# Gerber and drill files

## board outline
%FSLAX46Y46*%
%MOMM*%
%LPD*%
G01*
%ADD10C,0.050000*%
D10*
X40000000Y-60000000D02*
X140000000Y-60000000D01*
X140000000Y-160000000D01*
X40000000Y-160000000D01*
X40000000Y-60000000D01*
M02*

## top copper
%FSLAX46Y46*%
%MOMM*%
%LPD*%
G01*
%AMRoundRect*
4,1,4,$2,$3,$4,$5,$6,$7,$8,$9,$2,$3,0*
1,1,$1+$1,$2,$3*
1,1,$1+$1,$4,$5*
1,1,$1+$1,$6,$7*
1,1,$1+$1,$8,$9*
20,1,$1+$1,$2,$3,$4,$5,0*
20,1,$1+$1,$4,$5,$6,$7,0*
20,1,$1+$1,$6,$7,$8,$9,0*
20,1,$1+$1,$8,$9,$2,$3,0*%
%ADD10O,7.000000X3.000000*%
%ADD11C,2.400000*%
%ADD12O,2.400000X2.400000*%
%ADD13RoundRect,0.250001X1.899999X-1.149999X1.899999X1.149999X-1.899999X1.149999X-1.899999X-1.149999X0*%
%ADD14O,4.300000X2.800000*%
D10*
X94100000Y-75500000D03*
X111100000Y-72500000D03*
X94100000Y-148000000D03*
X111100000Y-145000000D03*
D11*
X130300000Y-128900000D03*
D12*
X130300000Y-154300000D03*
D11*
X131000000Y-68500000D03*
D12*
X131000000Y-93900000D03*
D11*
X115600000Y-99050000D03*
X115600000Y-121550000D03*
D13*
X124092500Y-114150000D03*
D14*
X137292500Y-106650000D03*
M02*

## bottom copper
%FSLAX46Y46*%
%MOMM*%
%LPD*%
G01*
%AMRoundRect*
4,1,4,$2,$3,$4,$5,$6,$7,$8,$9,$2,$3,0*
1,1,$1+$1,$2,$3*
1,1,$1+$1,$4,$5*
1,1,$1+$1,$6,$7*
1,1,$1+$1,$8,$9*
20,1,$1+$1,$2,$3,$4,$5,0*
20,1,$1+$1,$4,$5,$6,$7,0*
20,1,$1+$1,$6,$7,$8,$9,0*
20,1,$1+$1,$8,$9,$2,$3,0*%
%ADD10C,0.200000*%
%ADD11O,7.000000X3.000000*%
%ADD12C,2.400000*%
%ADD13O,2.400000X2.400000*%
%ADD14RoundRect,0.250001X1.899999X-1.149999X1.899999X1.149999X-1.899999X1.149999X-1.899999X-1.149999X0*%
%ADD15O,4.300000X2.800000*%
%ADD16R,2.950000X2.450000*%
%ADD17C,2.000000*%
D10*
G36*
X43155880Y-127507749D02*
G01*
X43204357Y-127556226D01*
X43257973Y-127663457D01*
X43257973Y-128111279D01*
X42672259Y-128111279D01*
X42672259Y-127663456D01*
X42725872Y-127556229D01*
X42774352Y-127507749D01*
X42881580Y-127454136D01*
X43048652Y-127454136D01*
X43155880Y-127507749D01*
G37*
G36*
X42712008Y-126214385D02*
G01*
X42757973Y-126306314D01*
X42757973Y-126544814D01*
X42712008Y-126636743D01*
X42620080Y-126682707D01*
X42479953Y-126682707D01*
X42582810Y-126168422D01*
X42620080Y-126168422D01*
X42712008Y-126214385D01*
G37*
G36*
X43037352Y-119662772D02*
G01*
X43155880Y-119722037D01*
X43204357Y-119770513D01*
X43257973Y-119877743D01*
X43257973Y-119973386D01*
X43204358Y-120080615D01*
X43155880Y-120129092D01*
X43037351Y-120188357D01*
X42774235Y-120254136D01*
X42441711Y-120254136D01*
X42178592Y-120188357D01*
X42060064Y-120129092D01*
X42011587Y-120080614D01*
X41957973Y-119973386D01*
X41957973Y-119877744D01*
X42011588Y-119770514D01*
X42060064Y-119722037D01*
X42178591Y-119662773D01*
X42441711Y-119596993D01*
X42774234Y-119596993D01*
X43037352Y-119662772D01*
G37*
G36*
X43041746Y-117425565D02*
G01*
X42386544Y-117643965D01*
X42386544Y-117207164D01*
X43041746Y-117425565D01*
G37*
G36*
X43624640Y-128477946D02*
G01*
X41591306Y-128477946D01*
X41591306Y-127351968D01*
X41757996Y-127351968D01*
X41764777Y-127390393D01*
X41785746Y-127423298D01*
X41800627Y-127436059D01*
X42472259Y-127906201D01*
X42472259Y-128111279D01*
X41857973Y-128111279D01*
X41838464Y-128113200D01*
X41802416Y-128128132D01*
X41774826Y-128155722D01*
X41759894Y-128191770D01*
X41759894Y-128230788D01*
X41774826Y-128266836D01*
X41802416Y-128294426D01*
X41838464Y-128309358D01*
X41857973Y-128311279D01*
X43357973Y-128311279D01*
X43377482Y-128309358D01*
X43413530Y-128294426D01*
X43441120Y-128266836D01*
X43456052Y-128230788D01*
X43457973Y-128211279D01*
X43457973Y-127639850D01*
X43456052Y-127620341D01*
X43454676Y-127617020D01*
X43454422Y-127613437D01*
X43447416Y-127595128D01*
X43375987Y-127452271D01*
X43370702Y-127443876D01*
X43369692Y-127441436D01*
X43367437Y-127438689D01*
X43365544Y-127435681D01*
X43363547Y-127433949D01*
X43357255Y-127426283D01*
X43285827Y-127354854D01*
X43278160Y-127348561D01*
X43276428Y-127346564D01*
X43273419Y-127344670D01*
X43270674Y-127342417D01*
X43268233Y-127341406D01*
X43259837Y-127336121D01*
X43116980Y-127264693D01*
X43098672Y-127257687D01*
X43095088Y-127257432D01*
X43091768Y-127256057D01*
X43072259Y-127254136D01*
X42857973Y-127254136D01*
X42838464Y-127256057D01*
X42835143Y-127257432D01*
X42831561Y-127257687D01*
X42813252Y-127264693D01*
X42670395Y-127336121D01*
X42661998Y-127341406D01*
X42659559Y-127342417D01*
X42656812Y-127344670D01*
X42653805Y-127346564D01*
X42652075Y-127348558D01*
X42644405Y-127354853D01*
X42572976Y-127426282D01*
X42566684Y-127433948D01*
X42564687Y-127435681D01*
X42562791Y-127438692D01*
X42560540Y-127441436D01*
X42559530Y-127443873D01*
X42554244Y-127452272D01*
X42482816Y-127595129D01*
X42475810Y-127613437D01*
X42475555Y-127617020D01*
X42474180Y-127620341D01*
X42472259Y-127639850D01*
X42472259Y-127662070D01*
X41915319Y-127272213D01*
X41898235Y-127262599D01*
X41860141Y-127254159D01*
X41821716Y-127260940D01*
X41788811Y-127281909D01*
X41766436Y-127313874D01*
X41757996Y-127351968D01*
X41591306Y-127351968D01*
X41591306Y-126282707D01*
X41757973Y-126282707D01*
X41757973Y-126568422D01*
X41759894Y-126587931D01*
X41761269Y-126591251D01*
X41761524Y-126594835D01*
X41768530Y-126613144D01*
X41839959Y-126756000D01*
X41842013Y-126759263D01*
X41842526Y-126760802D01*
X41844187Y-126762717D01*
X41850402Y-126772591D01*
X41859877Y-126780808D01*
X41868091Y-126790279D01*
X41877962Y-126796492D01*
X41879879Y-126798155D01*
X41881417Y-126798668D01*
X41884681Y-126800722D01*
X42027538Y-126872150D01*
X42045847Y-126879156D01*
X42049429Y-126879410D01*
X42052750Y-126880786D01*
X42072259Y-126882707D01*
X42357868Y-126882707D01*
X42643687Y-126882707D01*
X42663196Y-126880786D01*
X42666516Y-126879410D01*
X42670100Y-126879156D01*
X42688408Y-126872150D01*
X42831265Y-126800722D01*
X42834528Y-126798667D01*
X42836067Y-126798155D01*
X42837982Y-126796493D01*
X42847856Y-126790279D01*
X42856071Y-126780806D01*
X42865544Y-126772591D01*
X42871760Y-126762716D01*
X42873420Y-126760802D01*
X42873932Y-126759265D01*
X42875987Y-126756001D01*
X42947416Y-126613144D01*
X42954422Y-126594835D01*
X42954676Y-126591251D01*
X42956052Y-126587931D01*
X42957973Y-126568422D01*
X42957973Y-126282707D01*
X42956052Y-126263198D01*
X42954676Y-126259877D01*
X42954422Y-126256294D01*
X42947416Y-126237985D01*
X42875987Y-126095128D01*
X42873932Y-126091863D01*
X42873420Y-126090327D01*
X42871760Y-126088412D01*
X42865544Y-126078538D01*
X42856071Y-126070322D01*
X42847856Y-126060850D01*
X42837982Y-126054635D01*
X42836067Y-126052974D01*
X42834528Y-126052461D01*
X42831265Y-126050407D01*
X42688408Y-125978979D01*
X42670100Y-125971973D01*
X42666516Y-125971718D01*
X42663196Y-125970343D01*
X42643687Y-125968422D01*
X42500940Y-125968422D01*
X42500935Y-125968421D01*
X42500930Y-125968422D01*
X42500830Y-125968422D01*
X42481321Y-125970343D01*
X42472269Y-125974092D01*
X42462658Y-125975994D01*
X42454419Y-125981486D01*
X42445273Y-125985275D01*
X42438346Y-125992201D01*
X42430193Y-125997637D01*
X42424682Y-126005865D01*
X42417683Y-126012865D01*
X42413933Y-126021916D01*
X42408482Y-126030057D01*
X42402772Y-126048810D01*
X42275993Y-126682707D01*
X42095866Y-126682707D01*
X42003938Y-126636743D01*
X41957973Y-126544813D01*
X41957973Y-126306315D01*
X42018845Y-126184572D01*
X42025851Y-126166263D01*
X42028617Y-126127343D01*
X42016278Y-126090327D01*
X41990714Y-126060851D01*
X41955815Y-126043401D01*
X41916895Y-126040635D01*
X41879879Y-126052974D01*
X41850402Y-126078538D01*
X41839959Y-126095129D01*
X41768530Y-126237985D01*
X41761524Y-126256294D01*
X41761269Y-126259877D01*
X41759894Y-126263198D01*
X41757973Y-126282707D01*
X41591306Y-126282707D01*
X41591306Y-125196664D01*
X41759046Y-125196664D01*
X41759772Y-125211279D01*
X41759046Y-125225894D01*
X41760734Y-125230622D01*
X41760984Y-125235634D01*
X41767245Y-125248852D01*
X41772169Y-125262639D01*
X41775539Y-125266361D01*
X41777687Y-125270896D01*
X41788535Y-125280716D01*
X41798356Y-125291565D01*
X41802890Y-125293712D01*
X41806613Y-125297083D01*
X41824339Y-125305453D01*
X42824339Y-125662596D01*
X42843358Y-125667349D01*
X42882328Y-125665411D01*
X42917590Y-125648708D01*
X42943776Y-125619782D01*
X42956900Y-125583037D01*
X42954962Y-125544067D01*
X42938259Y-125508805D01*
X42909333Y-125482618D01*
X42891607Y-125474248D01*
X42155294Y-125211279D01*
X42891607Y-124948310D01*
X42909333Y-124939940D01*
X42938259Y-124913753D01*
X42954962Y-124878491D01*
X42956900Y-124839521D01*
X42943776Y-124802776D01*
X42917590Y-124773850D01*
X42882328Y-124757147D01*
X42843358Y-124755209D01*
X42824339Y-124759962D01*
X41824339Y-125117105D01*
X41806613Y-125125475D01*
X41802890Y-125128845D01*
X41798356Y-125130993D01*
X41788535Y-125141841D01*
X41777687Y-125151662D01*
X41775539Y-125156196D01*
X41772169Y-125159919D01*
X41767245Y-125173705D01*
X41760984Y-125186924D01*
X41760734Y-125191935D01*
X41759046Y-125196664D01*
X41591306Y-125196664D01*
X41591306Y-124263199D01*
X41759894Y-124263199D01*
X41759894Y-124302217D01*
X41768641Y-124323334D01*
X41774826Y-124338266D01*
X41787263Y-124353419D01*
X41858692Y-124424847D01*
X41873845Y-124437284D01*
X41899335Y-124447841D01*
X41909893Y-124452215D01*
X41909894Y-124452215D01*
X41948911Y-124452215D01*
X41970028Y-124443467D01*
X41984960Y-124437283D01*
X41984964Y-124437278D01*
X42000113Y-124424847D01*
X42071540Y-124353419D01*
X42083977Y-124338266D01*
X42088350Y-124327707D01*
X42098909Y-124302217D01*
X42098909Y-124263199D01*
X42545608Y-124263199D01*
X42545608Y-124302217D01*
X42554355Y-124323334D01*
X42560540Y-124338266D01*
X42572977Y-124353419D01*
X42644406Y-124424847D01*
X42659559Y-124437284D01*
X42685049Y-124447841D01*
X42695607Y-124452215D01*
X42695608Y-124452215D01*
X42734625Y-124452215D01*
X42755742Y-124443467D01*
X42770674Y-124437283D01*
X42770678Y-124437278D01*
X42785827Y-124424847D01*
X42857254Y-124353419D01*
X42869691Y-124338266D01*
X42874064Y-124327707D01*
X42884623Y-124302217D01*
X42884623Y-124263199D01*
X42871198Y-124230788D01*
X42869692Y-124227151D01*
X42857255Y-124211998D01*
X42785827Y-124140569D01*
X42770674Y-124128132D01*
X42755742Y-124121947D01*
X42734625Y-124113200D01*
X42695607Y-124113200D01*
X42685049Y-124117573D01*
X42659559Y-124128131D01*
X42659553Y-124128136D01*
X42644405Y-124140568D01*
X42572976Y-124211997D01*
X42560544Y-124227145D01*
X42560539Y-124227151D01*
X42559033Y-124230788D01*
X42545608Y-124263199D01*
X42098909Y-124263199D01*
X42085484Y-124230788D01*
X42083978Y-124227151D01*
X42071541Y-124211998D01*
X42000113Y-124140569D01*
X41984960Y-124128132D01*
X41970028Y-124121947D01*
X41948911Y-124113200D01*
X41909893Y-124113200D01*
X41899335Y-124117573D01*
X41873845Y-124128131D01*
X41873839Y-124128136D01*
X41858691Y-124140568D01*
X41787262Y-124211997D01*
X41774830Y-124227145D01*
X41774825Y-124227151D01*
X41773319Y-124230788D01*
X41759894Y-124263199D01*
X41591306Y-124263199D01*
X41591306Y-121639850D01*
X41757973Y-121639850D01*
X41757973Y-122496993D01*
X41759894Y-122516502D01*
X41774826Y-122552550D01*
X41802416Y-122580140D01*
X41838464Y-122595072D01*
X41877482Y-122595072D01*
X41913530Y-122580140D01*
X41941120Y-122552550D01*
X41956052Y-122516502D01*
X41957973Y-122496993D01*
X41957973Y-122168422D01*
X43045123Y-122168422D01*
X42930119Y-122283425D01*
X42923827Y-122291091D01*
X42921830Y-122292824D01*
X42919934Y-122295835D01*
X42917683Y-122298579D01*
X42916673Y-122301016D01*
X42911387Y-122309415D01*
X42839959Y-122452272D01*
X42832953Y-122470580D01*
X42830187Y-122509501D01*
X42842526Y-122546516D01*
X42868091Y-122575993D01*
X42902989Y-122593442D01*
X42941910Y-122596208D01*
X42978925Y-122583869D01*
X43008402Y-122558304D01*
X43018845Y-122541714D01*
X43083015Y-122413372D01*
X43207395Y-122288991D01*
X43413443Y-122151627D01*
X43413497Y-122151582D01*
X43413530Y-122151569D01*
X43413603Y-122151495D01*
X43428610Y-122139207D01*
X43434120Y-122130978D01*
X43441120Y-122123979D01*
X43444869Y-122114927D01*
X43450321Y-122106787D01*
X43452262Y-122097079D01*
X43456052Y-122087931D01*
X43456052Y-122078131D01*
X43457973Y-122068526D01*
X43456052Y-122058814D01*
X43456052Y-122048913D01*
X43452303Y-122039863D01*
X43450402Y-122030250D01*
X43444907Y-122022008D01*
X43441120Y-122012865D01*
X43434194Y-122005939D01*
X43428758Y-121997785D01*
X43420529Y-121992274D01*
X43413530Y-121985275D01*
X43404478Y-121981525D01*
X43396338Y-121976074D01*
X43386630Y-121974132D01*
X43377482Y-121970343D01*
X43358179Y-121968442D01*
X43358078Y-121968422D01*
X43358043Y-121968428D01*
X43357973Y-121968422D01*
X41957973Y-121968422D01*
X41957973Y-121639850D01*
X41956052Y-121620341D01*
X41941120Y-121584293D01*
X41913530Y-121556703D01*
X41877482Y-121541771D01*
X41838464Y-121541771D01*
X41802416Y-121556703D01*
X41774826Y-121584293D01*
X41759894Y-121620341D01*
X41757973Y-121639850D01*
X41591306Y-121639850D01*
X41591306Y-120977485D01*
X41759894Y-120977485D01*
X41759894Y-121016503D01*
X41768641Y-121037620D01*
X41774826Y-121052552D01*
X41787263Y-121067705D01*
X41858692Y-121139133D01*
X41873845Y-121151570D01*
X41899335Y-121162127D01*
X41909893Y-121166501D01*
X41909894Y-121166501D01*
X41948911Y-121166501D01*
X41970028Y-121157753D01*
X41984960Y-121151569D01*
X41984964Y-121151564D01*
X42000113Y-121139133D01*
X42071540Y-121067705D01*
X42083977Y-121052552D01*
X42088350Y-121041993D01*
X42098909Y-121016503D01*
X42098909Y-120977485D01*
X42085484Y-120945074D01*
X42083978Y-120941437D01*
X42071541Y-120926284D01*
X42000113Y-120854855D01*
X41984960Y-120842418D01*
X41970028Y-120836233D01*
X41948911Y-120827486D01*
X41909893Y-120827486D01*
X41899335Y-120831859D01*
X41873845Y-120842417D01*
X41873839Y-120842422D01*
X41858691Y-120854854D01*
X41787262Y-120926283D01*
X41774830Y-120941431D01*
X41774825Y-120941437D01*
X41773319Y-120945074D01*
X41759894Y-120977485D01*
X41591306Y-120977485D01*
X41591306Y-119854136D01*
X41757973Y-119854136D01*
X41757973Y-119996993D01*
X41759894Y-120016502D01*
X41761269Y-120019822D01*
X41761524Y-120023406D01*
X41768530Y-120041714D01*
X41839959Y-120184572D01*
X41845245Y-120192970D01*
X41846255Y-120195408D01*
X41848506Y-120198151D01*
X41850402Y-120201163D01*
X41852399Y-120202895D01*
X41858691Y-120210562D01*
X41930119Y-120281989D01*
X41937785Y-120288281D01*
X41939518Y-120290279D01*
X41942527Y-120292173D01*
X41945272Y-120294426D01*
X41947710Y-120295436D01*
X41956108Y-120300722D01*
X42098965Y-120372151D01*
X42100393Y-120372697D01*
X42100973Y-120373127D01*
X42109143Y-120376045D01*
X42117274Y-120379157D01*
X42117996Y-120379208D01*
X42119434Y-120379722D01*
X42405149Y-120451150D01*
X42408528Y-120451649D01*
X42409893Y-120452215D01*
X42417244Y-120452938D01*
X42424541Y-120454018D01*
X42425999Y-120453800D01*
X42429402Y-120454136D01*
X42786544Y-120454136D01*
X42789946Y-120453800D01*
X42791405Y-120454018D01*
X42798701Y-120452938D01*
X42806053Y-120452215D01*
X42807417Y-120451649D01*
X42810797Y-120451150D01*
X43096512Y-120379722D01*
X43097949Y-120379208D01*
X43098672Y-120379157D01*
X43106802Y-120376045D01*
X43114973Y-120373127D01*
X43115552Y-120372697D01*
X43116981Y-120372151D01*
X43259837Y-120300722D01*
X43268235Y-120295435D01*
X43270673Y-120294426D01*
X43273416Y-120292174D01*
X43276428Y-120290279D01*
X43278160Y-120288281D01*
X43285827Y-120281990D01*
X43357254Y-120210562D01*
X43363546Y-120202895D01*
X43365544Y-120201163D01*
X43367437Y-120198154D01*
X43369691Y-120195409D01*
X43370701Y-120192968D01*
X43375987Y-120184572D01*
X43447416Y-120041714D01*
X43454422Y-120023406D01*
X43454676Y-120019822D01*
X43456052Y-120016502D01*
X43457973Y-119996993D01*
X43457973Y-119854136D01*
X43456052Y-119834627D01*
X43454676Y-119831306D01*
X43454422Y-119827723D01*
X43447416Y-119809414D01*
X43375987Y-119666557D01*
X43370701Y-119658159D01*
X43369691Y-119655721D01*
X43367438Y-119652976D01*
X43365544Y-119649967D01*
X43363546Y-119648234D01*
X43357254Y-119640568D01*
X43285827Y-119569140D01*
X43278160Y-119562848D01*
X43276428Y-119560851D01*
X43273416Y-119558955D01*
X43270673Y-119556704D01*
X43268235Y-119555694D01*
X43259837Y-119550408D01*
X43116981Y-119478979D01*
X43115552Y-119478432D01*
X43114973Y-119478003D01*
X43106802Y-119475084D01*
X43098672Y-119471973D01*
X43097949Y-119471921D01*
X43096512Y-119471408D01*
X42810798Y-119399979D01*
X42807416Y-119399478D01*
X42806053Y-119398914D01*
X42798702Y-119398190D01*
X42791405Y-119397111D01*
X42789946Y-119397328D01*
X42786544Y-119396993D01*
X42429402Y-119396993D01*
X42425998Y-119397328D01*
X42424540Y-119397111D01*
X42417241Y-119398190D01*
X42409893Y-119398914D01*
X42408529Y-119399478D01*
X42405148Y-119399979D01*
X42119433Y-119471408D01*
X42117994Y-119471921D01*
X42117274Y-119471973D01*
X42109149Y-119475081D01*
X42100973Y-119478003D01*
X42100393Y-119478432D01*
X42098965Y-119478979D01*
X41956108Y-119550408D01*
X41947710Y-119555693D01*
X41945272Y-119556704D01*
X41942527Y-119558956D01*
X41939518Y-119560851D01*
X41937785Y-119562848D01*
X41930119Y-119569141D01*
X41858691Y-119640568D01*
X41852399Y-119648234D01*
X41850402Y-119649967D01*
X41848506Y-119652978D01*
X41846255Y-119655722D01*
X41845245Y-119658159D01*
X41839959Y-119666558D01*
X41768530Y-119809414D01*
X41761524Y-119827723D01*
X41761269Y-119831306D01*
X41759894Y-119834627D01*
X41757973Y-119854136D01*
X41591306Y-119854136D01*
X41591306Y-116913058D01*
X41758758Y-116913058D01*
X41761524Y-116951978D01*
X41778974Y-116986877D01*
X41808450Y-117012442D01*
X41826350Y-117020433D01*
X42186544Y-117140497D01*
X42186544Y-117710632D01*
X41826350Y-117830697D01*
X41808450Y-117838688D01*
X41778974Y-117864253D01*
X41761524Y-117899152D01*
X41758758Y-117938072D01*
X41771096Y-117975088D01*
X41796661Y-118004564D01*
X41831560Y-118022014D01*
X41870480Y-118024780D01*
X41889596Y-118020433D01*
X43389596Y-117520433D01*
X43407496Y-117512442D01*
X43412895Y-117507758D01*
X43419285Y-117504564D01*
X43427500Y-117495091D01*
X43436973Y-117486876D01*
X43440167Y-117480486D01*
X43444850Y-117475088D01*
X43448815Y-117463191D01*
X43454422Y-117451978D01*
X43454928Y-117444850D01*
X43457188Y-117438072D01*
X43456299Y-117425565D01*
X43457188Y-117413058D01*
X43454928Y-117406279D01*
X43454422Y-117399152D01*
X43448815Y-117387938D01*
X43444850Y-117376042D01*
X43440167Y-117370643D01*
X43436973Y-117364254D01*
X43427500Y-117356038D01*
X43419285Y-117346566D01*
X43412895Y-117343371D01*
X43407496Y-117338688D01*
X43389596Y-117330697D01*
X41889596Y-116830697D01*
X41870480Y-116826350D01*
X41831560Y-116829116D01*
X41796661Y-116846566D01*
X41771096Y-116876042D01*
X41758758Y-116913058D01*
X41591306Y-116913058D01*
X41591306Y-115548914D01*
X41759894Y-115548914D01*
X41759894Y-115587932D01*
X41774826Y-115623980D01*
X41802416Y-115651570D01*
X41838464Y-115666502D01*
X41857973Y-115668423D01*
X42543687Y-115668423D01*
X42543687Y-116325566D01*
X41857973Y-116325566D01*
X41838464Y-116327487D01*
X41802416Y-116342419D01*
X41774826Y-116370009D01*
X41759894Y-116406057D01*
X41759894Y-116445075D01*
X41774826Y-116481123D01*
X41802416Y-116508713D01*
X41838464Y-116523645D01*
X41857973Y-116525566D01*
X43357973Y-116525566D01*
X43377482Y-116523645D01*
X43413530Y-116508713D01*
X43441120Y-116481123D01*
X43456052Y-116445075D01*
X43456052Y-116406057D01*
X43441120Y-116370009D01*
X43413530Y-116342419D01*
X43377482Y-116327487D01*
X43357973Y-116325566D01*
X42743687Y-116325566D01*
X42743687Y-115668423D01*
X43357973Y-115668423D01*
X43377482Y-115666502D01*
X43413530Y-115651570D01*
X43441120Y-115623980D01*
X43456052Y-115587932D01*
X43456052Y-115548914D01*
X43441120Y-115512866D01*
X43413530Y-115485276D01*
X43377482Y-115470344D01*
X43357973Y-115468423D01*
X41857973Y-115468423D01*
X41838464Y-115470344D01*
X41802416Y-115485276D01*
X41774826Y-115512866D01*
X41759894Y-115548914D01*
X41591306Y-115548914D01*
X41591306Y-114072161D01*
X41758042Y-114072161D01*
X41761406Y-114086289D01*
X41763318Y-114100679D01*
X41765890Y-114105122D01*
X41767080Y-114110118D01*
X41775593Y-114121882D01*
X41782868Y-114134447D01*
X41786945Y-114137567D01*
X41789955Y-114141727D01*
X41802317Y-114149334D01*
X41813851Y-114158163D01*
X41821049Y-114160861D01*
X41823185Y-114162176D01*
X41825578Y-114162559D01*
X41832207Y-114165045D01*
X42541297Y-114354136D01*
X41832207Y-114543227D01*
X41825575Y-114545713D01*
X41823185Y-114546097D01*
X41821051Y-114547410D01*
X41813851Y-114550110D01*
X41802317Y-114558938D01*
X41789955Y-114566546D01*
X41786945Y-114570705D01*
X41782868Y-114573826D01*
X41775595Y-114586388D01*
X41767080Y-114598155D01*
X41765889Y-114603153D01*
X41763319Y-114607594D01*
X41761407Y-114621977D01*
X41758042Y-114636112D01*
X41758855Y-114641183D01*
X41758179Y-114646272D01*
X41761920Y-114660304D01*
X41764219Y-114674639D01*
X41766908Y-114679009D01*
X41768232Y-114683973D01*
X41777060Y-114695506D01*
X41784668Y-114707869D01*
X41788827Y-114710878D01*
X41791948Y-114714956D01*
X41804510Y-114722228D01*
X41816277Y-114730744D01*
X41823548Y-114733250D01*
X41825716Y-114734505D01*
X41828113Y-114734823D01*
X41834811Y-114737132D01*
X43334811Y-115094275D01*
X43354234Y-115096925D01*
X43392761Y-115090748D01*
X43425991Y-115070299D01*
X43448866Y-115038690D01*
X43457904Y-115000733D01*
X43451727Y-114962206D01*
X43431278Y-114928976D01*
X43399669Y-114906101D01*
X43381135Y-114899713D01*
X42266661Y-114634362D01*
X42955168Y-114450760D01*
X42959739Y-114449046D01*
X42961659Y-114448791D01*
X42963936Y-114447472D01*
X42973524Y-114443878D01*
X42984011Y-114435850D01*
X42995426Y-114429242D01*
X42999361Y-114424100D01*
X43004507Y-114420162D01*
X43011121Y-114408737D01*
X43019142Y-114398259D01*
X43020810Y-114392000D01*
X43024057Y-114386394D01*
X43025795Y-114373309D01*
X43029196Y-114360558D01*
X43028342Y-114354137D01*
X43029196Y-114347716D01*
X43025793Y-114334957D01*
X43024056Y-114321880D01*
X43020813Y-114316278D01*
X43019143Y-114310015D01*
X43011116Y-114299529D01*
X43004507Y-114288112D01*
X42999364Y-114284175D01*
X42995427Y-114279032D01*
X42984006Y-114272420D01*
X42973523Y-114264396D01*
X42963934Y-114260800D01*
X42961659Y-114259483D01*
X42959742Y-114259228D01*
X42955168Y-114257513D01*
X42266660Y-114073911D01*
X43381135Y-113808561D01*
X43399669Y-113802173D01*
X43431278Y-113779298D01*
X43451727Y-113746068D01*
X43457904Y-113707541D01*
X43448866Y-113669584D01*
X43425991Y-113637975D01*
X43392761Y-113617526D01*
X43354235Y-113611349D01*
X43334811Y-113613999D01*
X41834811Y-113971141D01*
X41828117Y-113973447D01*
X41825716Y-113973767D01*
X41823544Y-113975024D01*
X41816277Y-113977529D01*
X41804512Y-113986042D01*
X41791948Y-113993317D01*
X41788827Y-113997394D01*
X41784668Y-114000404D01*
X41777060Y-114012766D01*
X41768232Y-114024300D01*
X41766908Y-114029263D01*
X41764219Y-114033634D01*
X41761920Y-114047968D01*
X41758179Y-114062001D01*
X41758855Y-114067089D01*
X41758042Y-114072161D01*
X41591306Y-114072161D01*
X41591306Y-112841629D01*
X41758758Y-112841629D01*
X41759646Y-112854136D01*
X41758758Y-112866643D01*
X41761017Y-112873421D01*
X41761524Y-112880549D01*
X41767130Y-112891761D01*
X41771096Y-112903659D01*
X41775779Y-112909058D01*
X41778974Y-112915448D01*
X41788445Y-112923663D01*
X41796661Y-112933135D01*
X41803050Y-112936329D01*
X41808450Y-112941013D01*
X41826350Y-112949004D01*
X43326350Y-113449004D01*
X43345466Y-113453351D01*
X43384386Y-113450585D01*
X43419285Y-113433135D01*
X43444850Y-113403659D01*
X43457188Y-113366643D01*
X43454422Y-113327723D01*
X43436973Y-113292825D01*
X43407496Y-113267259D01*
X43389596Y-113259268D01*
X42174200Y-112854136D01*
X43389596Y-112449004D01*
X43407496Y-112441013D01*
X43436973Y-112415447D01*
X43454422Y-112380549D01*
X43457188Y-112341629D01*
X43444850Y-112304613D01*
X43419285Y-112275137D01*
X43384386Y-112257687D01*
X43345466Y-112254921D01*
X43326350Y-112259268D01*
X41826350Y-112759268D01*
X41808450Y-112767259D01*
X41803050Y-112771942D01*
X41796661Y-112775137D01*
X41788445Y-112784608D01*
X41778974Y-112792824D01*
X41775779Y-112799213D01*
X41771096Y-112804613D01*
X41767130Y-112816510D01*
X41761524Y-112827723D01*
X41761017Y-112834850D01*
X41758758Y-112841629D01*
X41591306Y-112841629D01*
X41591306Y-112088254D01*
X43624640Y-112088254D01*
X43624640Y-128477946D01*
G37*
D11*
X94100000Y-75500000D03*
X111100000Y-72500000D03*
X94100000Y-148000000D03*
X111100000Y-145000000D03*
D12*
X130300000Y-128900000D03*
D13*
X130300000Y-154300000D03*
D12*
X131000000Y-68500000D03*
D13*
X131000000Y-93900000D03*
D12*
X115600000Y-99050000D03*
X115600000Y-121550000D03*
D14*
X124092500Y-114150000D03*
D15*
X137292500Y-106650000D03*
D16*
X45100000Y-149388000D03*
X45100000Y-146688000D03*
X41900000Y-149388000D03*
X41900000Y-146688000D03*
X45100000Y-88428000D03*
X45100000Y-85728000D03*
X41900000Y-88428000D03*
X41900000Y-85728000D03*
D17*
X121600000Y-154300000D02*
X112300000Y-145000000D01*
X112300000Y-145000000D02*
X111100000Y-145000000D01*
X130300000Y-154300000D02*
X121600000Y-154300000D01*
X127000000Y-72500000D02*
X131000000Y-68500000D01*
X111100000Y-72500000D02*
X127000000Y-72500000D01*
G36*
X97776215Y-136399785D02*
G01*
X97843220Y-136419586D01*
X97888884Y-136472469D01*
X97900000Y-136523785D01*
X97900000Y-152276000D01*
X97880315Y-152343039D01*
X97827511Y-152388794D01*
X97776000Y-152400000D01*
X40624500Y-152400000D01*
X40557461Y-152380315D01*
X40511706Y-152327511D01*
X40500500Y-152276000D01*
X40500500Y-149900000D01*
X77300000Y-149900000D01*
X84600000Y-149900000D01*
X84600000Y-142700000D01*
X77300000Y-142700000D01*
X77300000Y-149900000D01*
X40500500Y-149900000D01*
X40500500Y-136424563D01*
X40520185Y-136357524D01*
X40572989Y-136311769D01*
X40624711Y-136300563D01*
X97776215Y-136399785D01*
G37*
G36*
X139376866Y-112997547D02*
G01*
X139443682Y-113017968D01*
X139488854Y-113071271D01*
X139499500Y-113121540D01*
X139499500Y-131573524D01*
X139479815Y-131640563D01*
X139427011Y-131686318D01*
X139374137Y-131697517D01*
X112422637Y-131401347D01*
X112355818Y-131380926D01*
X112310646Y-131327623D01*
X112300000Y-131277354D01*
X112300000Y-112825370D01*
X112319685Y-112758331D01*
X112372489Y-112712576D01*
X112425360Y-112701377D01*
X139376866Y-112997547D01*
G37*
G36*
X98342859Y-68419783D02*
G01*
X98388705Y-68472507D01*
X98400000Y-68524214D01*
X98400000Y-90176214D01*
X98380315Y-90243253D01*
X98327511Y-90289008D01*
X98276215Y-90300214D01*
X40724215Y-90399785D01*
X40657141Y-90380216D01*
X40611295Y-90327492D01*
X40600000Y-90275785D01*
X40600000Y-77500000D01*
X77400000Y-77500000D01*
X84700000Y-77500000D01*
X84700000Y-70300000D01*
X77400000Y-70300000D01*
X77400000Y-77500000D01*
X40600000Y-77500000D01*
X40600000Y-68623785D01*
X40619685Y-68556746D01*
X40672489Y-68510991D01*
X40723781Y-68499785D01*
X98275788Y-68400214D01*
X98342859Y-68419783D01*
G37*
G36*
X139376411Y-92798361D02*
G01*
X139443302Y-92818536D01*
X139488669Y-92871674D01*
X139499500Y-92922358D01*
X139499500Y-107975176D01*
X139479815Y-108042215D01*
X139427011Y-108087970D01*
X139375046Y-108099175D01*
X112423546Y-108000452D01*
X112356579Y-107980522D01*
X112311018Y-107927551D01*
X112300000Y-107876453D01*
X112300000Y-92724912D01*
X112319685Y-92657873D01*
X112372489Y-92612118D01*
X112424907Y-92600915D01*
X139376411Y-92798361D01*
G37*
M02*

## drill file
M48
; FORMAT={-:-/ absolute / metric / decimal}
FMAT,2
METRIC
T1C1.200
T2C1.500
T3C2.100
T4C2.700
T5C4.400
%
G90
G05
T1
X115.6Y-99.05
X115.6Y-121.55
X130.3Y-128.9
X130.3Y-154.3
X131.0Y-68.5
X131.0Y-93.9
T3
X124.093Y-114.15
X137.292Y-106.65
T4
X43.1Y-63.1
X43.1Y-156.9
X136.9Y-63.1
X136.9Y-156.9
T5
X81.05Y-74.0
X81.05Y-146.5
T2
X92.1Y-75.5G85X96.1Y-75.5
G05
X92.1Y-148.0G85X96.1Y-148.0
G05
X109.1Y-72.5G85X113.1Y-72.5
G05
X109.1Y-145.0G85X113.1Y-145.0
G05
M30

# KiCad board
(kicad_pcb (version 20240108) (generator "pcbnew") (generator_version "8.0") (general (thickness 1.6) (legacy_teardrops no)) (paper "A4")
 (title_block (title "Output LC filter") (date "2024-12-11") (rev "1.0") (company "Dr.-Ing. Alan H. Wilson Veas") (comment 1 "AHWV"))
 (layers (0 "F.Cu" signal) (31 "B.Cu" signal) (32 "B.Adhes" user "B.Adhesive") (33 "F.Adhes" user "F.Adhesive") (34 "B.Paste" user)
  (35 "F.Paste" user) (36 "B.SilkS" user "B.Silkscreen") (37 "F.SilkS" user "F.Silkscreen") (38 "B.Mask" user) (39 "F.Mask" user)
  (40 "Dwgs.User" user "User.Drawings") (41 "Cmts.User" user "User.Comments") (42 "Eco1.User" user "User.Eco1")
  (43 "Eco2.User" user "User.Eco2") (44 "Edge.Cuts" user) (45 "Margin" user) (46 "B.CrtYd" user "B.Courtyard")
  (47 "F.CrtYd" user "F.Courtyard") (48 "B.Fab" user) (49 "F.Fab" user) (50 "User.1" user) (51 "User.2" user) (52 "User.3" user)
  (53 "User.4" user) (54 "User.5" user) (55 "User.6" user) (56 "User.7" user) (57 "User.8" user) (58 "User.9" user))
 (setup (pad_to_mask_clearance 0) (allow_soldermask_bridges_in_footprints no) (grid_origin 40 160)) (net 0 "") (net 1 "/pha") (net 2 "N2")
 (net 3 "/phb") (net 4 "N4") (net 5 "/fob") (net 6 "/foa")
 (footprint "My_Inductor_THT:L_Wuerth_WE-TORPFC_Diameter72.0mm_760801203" (layer "F.Cu") (at 81.05 74)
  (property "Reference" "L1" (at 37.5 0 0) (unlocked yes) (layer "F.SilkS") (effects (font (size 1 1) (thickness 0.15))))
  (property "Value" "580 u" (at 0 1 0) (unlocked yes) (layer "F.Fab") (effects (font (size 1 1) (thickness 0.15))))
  (pad "" np_thru_hole circle (at 0 0) (size 4.4 4.4) (drill 4.4) (layers "F&B.Cu" "*.Mask"))
  (pad "1" thru_hole oval (at 13.05 1.5) (size 7 3) (drill oval 5.5 1.5) (layers "*.Cu" "*.Mask") (remove_unused_layers no) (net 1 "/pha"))
  (pad "2" thru_hole oval (at 30.05 -1.5) (size 7 3) (drill oval 5.5 1.5) (layers "*.Cu" "*.Mask") (remove_unused_layers no) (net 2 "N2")))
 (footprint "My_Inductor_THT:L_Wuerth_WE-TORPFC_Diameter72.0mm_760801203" (layer "F.Cu") (at 81.05 146.5)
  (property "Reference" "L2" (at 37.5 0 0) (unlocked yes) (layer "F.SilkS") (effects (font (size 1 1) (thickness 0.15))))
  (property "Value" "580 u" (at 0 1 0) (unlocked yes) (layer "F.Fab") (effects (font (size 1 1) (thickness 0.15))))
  (pad "" np_thru_hole circle (at 0 0) (size 4.4 4.4) (drill 4.4) (layers "F&B.Cu" "*.Mask"))
  (pad "1" thru_hole oval (at 13.05 1.5) (size 7 3) (drill oval 5.5 1.5) (layers "*.Cu" "*.Mask") (remove_unused_layers no) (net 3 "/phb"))
  (pad "2" thru_hole oval (at 30.05 -1.5) (size 7 3) (drill oval 5.5 1.5) (layers "*.Cu" "*.Mask") (remove_unused_layers no) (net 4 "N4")))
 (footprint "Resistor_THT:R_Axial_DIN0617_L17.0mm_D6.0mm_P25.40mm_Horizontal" (layer "F.Cu") (at 130.3 128.9 -90)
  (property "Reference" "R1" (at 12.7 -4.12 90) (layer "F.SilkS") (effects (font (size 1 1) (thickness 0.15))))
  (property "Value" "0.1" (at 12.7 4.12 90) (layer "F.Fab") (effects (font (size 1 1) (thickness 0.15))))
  (pad "1" thru_hole circle (at 0 0 270) (size 2.4 2.4) (drill 1.2) (layers "*.Cu" "*.Mask") (remove_unused_layers no) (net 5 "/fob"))
  (pad "2" thru_hole oval (at 25.4 0 270) (size 2.4 2.4) (drill 1.2) (layers "*.Cu" "*.Mask") (remove_unused_layers no) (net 4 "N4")))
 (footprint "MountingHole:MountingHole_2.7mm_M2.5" (layer "F.Cu") (at 136.9 63.1 180)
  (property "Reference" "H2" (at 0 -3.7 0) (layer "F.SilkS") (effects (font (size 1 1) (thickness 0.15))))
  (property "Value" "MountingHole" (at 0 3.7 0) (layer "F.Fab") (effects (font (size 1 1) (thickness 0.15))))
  (pad "" np_thru_hole circle (at 0 0 180) (size 2.7 2.7) (drill 2.7) (layers "*.Cu" "*.Mask")))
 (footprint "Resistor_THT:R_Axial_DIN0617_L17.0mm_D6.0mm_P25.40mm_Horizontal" (layer "F.Cu") (at 131 68.5 -90)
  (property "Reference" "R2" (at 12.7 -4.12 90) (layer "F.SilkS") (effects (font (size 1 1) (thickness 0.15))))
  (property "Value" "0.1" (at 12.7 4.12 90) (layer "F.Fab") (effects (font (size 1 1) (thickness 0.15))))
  (pad "1" thru_hole circle (at 0 0 270) (size 2.4 2.4) (drill 1.2) (layers "*.Cu" "*.Mask") (remove_unused_layers no) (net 2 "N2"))
  (pad "2" thru_hole oval (at 25.4 0 270) (size 2.4 2.4) (drill 1.2) (layers "*.Cu" "*.Mask") (remove_unused_layers no) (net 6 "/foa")))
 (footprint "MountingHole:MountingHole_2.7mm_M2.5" (layer "F.Cu") (at 43.1 63.1 180)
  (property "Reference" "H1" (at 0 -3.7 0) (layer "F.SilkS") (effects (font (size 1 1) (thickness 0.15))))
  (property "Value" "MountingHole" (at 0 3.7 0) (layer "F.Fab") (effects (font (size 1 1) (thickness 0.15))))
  (pad "" np_thru_hole circle (at 0 0 180) (size 2.7 2.7) (drill 2.7) (layers "*.Cu" "*.Mask")))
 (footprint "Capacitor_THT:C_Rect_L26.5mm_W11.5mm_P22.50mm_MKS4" (layer "F.Cu") (at 115.6 99.05 -90)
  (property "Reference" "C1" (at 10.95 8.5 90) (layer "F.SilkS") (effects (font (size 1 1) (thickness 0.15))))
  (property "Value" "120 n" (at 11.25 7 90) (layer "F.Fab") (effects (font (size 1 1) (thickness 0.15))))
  (pad "1" thru_hole circle (at 0 0 270) (size 2.4 2.4) (drill 1.2) (layers "*.Cu" "*.Mask") (remove_unused_layers no) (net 6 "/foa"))
  (pad "2" thru_hole circle (at 22.5 0 270) (size 2.4 2.4) (drill 1.2) (layers "*.Cu" "*.Mask") (remove_unused_layers no) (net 5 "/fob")))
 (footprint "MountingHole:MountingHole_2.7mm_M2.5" (layer "F.Cu") (at 136.9 156.9)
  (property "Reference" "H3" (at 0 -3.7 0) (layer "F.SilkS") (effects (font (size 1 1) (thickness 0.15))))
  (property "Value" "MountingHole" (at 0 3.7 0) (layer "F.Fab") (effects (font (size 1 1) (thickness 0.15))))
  (pad "" np_thru_hole circle (at 0 0) (size 2.7 2.7) (drill 2.7) (layers "*.Cu" "*.Mask")))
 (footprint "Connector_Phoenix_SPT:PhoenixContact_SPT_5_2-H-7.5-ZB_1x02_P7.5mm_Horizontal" (layer "F.Cu") (at 124.0925 114.15 90)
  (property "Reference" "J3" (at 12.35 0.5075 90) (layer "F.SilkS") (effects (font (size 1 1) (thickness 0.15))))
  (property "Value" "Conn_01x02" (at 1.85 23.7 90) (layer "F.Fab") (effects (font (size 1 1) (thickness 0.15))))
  (pad "1" thru_hole roundrect (at 0 0 90) (size 2.8 4.3) (drill 2.1) (layers "*.Cu" "*.Mask") (remove_unused_layers no)
   (roundrect_rratio 0.089286) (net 5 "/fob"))
  (pad "2" thru_hole oval (at 7.5 13.2 90) (size 2.8 4.3) (drill 2.1) (layers "*.Cu" "*.Mask") (remove_unused_layers no) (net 6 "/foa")))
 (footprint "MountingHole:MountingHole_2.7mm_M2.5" (layer "F.Cu") (at 43.1 156.9)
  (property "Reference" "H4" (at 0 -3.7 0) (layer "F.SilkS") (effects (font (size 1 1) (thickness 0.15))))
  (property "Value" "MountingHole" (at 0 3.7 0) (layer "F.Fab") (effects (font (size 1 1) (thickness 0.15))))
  (pad "" np_thru_hole circle (at 0 0) (size 2.7 2.7) (drill 2.7) (layers "*.Cu" "*.Mask")))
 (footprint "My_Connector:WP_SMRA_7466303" (layer "B.Cu") (at 43.5 148.038 180)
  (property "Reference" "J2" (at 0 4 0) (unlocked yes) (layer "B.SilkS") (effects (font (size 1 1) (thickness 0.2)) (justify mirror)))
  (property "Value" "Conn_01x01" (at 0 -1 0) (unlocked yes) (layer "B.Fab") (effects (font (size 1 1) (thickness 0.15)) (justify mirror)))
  (pad "1" smd rect (at -1.6 -1.35 180) (size 2.95 2.45) (layers "B.Cu" "B.Paste" "B.Mask") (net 3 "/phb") (solder_mask_margin 0.125)
   (solder_paste_margin -0.2) (thermal_bridge_angle 45))
  (pad "1" smd rect (at -1.6 1.35 180) (size 2.95 2.45) (layers "B.Cu" "B.Paste" "B.Mask") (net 3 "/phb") (solder_mask_margin 0.125)
   (solder_paste_margin -0.2) (thermal_bridge_angle 45))
  (pad "1" smd rect (at 1.6 -1.35 180) (size 2.95 2.45) (layers "B.Cu" "B.Paste" "B.Mask") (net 3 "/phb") (solder_mask_margin 0.125)
   (solder_paste_margin -0.2) (thermal_bridge_angle 45))
  (pad "1" smd rect (at 1.6 1.35 180) (size 2.95 2.45) (layers "B.Cu" "B.Paste" "B.Mask") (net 3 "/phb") (solder_mask_margin 0.125)
   (solder_paste_margin -0.2) (thermal_bridge_angle 45)))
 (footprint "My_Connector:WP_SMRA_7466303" (layer "B.Cu") (at 43.5 87.078 180)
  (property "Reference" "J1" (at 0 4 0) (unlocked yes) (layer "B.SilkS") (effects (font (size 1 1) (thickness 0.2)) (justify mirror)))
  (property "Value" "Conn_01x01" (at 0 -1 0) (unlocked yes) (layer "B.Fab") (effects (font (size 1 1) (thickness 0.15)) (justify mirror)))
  (pad "1" smd rect (at -1.6 -1.35 180) (size 2.95 2.45) (layers "B.Cu" "B.Paste" "B.Mask") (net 1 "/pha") (solder_mask_margin 0.125)
   (solder_paste_margin -0.2) (thermal_bridge_angle 45))
  (pad "1" smd rect (at -1.6 1.35 180) (size 2.95 2.45) (layers "B.Cu" "B.Paste" "B.Mask") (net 1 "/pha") (solder_mask_margin 0.125)
   (solder_paste_margin -0.2) (thermal_bridge_angle 45))
  (pad "1" smd rect (at 1.6 -1.35 180) (size 2.95 2.45) (layers "B.Cu" "B.Paste" "B.Mask") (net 1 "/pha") (solder_mask_margin 0.125)
   (solder_paste_margin -0.2) (thermal_bridge_angle 45))
  (pad "1" smd rect (at 1.6 1.35 180) (size 2.95 2.45) (layers "B.Cu" "B.Paste" "B.Mask") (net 1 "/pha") (solder_mask_margin 0.125)
   (solder_paste_margin -0.2) (thermal_bridge_angle 45)))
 (gr_rect (start 40 60) (end 140 160) (stroke (width 0.05) (type default)) (fill none) (layer "Edge.Cuts"))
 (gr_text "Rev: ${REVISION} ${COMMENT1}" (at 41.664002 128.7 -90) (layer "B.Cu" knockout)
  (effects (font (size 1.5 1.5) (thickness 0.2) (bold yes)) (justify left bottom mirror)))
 (segment (start 121.6 154.3) (end 112.3 145) (width 2) (layer "B.Cu") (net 4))
 (segment (start 112.3 145) (end 111.1 145) (width 2) (layer "B.Cu") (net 4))
 (segment (start 130.3 154.3) (end 121.6 154.3) (width 2) (layer "B.Cu") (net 4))
 (segment (start 127 72.5) (end 131 68.5) (width 2) (layer "B.Cu") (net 2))
 (segment (start 111.1 72.5) (end 127 72.5) (width 2) (layer "B.Cu") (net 2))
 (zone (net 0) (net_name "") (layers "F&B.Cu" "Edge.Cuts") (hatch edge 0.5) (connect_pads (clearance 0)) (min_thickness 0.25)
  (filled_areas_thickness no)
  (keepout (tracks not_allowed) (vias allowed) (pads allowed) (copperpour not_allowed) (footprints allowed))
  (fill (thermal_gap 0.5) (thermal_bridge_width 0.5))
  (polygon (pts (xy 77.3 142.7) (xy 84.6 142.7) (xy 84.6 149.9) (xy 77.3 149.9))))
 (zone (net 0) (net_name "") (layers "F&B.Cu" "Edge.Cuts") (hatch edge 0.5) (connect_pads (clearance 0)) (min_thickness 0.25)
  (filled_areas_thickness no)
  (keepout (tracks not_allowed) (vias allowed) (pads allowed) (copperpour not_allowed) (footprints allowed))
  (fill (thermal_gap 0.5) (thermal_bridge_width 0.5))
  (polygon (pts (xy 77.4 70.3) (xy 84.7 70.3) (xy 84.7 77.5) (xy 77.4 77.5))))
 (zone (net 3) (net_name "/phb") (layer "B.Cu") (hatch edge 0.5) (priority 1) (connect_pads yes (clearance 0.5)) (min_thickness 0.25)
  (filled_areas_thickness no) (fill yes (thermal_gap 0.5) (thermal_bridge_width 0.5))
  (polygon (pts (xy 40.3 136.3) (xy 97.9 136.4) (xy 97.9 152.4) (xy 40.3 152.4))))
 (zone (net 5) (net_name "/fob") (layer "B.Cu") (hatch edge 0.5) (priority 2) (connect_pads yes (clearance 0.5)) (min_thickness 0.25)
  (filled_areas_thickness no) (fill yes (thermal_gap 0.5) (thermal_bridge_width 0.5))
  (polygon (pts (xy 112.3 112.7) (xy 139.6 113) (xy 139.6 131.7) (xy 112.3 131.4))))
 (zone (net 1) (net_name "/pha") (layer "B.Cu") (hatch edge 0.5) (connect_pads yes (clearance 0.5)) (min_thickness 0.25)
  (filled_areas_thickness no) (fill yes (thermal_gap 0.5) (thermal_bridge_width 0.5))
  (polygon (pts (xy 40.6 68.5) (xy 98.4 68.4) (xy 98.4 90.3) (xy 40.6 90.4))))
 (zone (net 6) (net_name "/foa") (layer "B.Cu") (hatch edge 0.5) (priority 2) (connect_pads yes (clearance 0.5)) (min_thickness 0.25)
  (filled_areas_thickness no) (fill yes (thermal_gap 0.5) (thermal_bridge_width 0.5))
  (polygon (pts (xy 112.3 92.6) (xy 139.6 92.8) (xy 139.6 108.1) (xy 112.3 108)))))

